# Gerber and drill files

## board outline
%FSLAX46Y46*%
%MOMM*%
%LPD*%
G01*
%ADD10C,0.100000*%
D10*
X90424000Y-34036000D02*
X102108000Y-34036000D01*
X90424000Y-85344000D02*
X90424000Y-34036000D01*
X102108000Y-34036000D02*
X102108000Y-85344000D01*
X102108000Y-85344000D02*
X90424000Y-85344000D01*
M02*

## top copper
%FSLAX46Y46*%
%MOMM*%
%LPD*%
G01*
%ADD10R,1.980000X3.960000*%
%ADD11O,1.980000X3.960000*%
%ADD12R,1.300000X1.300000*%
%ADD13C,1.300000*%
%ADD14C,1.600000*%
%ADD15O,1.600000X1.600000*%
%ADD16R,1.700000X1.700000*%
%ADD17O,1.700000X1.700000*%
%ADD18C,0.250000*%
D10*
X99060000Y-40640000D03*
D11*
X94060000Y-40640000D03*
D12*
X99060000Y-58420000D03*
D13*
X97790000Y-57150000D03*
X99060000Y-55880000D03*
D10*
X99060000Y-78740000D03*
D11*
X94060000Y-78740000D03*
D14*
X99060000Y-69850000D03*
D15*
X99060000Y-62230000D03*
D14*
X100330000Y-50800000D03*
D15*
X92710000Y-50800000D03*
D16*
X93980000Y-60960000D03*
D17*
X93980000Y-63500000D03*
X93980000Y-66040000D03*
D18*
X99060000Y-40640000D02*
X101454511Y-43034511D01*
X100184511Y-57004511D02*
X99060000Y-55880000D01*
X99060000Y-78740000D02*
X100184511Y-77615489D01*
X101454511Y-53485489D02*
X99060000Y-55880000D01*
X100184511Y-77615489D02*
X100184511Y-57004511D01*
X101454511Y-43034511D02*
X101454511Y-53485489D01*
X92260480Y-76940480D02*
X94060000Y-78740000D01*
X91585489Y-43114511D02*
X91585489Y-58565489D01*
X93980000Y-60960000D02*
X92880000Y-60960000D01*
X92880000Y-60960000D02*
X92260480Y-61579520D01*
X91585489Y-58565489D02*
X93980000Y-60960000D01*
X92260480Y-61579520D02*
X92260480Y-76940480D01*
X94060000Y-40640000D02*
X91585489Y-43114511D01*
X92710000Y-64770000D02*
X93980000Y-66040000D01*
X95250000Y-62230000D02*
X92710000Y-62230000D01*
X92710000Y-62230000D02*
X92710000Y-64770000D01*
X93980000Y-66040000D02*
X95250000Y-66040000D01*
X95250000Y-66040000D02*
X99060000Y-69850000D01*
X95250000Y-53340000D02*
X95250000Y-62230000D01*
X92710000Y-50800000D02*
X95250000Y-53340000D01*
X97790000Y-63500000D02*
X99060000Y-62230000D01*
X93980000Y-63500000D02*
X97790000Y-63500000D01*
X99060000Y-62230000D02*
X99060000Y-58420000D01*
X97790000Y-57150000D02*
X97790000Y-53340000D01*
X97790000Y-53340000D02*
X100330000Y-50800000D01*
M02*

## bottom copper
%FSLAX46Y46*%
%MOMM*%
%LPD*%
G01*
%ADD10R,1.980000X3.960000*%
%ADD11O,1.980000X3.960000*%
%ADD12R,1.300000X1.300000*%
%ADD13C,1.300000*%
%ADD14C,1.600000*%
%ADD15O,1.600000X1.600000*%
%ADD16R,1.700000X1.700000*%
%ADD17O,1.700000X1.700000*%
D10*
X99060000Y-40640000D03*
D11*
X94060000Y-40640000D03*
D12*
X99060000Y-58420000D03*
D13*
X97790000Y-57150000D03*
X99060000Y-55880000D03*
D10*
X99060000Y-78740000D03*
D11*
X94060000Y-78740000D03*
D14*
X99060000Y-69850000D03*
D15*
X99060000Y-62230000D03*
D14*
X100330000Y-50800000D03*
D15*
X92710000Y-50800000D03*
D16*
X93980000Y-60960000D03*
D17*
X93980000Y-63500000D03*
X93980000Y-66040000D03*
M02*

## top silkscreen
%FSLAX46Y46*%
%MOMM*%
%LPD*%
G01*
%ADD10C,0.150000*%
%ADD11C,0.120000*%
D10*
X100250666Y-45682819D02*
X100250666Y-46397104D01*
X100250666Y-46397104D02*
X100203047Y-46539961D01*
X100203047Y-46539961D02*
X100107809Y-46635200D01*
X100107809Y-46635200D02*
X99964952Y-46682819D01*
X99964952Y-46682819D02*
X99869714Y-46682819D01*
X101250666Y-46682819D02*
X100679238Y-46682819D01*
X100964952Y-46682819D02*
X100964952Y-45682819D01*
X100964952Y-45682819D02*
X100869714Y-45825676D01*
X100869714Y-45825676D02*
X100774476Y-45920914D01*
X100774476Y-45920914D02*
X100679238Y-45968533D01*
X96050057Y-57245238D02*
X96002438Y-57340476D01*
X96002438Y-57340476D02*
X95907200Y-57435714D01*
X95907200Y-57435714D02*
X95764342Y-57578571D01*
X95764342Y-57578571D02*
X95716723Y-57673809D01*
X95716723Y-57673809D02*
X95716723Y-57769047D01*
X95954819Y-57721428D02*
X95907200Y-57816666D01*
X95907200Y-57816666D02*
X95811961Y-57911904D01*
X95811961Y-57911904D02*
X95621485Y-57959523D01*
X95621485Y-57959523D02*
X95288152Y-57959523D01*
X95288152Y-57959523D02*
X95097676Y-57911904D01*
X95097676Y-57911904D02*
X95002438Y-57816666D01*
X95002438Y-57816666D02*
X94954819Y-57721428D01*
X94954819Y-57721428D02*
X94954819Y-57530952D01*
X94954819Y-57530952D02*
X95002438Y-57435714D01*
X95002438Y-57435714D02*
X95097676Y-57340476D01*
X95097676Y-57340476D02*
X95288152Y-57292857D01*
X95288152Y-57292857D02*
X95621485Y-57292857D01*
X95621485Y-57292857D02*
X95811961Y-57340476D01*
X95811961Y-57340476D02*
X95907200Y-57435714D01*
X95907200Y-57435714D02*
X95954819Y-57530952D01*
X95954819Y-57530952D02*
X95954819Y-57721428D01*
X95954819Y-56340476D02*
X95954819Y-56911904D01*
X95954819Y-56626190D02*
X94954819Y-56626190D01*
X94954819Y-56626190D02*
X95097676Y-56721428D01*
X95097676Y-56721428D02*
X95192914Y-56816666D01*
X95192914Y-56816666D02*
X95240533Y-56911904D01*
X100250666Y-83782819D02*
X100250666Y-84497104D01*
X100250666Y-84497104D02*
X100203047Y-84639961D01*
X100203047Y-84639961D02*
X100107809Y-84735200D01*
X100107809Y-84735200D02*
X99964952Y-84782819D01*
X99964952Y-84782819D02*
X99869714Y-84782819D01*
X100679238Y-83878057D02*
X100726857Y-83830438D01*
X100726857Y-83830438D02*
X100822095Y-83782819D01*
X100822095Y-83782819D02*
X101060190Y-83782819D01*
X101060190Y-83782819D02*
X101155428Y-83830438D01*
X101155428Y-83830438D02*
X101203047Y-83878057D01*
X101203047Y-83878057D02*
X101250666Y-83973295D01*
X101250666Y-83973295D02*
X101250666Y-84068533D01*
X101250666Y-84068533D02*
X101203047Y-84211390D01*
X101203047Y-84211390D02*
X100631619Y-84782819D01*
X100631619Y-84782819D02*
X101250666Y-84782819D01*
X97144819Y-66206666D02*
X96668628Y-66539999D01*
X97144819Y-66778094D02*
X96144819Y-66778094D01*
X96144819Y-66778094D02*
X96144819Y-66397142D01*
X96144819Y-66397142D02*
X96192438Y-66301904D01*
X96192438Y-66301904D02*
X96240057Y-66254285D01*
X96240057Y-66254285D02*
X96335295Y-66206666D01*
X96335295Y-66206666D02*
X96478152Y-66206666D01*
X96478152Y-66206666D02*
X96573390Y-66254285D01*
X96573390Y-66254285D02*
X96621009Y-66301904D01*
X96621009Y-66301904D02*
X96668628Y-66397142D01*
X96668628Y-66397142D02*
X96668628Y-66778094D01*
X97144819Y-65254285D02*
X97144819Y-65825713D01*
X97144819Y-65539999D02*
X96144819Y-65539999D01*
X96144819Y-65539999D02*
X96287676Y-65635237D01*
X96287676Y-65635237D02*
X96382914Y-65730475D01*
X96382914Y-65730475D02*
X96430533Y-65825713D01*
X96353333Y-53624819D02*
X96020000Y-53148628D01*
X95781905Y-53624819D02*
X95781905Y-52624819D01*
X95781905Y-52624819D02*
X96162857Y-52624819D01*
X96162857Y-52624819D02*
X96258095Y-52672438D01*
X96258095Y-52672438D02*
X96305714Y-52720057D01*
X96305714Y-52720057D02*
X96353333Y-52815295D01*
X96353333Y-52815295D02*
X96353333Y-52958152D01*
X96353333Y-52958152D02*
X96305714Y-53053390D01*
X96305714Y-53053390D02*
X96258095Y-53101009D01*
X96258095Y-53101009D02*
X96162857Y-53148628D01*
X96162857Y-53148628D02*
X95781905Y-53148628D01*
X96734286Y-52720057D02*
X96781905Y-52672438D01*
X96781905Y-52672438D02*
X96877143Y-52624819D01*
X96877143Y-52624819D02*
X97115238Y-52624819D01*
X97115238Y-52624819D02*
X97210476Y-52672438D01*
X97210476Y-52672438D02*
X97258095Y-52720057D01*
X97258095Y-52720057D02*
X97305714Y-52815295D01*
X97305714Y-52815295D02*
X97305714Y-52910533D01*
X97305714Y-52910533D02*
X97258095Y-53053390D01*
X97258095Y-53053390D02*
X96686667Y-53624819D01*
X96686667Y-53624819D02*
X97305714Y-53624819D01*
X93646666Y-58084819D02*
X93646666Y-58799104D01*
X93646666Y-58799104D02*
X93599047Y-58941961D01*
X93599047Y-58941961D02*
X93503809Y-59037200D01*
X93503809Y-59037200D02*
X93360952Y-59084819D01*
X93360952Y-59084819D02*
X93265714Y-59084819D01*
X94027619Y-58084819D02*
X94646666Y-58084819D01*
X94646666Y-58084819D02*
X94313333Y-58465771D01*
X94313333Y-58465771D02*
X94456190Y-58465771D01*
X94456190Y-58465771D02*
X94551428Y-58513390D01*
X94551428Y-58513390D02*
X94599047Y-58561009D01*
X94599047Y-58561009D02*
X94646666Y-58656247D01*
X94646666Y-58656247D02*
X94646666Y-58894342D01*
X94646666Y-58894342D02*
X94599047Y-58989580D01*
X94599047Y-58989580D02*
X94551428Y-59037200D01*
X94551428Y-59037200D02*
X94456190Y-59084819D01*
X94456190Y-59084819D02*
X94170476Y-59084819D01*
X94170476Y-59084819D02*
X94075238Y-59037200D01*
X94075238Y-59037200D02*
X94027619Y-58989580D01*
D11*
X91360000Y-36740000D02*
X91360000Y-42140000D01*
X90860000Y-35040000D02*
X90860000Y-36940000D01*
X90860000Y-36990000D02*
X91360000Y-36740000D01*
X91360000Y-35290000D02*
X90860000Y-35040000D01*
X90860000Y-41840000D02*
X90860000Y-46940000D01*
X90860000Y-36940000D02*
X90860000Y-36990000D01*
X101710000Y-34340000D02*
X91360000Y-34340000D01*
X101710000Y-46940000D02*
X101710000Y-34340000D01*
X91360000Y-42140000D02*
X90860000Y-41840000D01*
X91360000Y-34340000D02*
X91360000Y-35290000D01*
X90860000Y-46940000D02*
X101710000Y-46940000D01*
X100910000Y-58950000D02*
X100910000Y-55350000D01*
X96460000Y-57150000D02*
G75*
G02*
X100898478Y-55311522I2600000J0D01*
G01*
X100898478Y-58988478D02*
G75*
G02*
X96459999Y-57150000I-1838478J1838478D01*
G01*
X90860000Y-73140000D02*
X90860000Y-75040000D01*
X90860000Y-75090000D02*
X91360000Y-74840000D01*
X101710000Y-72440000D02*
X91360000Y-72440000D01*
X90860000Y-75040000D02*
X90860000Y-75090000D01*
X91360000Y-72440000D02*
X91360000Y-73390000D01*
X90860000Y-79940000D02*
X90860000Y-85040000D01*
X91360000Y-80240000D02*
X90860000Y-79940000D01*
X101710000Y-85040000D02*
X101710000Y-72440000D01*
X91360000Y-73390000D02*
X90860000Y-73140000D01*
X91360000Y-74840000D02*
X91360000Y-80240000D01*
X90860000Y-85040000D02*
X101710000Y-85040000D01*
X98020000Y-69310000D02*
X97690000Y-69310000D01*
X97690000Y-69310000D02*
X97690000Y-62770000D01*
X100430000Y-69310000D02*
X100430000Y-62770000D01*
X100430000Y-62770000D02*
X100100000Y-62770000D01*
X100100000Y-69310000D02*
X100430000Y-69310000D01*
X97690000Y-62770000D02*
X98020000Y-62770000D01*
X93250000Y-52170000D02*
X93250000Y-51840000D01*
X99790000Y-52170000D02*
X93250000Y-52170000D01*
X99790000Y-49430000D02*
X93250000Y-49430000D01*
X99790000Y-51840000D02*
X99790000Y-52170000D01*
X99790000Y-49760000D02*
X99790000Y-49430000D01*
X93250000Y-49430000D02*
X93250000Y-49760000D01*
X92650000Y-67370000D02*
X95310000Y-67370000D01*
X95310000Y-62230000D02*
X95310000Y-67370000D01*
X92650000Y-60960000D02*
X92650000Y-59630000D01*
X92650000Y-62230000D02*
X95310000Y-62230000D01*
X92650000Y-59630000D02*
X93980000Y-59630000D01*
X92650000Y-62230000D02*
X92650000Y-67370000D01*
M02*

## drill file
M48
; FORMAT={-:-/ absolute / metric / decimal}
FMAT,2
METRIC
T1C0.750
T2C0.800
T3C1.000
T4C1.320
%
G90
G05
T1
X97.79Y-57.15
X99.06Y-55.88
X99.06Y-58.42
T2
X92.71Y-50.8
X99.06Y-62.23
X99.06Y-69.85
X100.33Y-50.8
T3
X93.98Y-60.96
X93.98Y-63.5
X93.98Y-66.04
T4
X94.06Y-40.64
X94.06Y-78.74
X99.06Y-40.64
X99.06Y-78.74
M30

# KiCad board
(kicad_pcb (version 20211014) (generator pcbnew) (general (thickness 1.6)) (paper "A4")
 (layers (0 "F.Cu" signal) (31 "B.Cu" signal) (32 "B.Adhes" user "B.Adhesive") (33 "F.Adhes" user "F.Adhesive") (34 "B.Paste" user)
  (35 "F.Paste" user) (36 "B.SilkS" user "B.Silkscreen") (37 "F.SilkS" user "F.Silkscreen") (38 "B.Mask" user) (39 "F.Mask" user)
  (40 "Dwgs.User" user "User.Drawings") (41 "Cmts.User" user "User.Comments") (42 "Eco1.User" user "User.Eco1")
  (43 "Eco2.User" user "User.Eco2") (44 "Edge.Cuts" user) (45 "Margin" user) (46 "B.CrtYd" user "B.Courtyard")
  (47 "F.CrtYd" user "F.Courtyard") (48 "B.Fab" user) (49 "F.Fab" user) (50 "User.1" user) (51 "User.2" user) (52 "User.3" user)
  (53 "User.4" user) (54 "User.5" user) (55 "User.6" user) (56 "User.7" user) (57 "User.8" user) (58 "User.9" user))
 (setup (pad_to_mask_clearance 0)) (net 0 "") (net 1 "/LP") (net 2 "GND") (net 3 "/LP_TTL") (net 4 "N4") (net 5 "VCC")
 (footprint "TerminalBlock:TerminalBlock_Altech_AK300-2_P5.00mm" (layer "F.Cu") (at 99.06 40.64 180)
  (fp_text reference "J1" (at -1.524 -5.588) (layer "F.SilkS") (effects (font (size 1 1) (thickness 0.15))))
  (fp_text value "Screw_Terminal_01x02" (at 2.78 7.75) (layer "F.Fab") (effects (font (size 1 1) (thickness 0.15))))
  (fp_line (start 7.7 3.9) (end 7.7 -1.5) (layer "F.SilkS") (width 0.12))
  (fp_line (start 8.2 5.6) (end 8.2 3.7) (layer "F.SilkS") (width 0.12))
  (fp_line (start 8.2 3.65) (end 7.7 3.9) (layer "F.SilkS") (width 0.12))
  (fp_line (start 7.7 5.35) (end 8.2 5.6) (layer "F.SilkS") (width 0.12))
  (fp_line (start 8.2 -1.2) (end 8.2 -6.3) (layer "F.SilkS") (width 0.12))
  (fp_line (start 8.2 3.7) (end 8.2 3.65) (layer "F.SilkS") (width 0.12))
  (fp_line (start -2.65 6.3) (end 7.7 6.3) (layer "F.SilkS") (width 0.12))
  (fp_line (start -2.65 -6.3) (end -2.65 6.3) (layer "F.SilkS") (width 0.12))
  (fp_line (start 7.7 -1.5) (end 8.2 -1.2) (layer "F.SilkS") (width 0.12))
  (fp_line (start 7.7 6.3) (end 7.7 5.35) (layer "F.SilkS") (width 0.12))
  (fp_line (start 8.2 -6.3) (end -2.65 -6.3) (layer "F.SilkS") (width 0.12))
  (pad "1" thru_hole rect (at 0 0 180) (size 1.98 3.96) (drill 1.32) (layers *.Cu *.Mask) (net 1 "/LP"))
  (pad "2" thru_hole oval (at 5 0 180) (size 1.98 3.96) (drill 1.32) (layers *.Cu *.Mask) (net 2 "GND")))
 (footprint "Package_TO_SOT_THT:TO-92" (layer "F.Cu") (at 99.06 58.42 90)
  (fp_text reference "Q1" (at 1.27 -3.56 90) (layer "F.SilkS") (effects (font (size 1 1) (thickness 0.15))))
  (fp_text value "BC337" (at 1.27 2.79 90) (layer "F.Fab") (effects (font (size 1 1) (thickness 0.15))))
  (fp_line (start -0.53 1.85) (end 3.07 1.85) (layer "F.SilkS") (width 0.12))
  (fp_arc (start 1.27 -2.6) (mid 3.672087 -0.994977) (end 3.108478 1.838478) (layer "F.SilkS") (width 0.12))
  (fp_arc (start -0.568478 1.838478) (mid -1.132087 -0.994977) (end 1.27 -2.6) (layer "F.SilkS") (width 0.12))
  (pad "1" thru_hole rect (at 0 0 90) (size 1.3 1.3) (drill 0.75) (layers *.Cu *.Mask) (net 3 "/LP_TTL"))
  (pad "2" thru_hole circle (at 1.27 -1.27 90) (size 1.3 1.3) (drill 0.75) (layers *.Cu *.Mask) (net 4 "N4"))
  (pad "3" thru_hole circle (at 2.54 0 90) (size 1.3 1.3) (drill 0.75) (layers *.Cu *.Mask) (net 1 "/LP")))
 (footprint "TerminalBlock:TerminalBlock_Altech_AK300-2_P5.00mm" (layer "F.Cu") (at 99.06 78.74 180)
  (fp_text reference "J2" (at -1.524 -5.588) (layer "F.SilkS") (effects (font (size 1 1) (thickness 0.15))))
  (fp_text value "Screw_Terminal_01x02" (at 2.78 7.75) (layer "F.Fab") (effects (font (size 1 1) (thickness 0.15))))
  (fp_line (start 8.2 5.6) (end 8.2 3.7) (layer "F.SilkS") (width 0.12))
  (fp_line (start 8.2 3.65) (end 7.7 3.9) (layer "F.SilkS") (width 0.12))
  (fp_line (start -2.65 6.3) (end 7.7 6.3) (layer "F.SilkS") (width 0.12))
  (fp_line (start 8.2 3.7) (end 8.2 3.65) (layer "F.SilkS") (width 0.12))
  (fp_line (start 7.7 6.3) (end 7.7 5.35) (layer "F.SilkS") (width 0.12))
  (fp_line (start 8.2 -1.2) (end 8.2 -6.3) (layer "F.SilkS") (width 0.12))
  (fp_line (start 7.7 -1.5) (end 8.2 -1.2) (layer "F.SilkS") (width 0.12))
  (fp_line (start -2.65 -6.3) (end -2.65 6.3) (layer "F.SilkS") (width 0.12))
  (fp_line (start 7.7 5.35) (end 8.2 5.6) (layer "F.SilkS") (width 0.12))
  (fp_line (start 7.7 3.9) (end 7.7 -1.5) (layer "F.SilkS") (width 0.12))
  (fp_line (start 8.2 -6.3) (end -2.65 -6.3) (layer "F.SilkS") (width 0.12))
  (pad "1" thru_hole rect (at 0 0 180) (size 1.98 3.96) (drill 1.32) (layers *.Cu *.Mask) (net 1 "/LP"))
  (pad "2" thru_hole oval (at 5 0 180) (size 1.98 3.96) (drill 1.32) (layers *.Cu *.Mask) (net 2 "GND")))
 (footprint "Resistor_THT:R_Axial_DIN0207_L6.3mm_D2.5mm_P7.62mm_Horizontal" (layer "F.Cu") (at 99.06 69.85 90)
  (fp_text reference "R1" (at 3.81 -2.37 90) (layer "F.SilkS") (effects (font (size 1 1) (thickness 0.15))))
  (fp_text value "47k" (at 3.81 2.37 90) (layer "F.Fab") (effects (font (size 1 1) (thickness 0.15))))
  (fp_line (start 0.54 -1.04) (end 0.54 -1.37) (layer "F.SilkS") (width 0.12))
  (fp_line (start 0.54 -1.37) (end 7.08 -1.37) (layer "F.SilkS") (width 0.12))
  (fp_line (start 0.54 1.37) (end 7.08 1.37) (layer "F.SilkS") (width 0.12))
  (fp_line (start 7.08 1.37) (end 7.08 1.04) (layer "F.SilkS") (width 0.12))
  (fp_line (start 0.54 1.04) (end 0.54 1.37) (layer "F.SilkS") (width 0.12))
  (fp_line (start 7.08 -1.37) (end 7.08 -1.04) (layer "F.SilkS") (width 0.12))
  (pad "1" thru_hole circle (at 0 0 90) (size 1.6 1.6) (drill 0.8) (layers *.Cu *.Mask) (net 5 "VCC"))
  (pad "2" thru_hole oval (at 7.62 0 90) (size 1.6 1.6) (drill 0.8) (layers *.Cu *.Mask) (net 3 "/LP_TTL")))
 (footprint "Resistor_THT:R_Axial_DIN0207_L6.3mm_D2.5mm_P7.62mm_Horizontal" (layer "F.Cu") (at 100.33 50.8 180)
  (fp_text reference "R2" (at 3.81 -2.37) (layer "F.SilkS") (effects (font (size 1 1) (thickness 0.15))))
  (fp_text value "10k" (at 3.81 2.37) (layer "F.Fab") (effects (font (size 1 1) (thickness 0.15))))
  (fp_line (start 7.08 -1.37) (end 7.08 -1.04) (layer "F.SilkS") (width 0.12))
  (fp_line (start 0.54 -1.37) (end 7.08 -1.37) (layer "F.SilkS") (width 0.12))
  (fp_line (start 0.54 1.37) (end 7.08 1.37) (layer "F.SilkS") (width 0.12))
  (fp_line (start 0.54 -1.04) (end 0.54 -1.37) (layer "F.SilkS") (width 0.12))
  (fp_line (start 0.54 1.04) (end 0.54 1.37) (layer "F.SilkS") (width 0.12))
  (fp_line (start 7.08 1.37) (end 7.08 1.04) (layer "F.SilkS") (width 0.12))
  (pad "1" thru_hole circle (at 0 0 180) (size 1.6 1.6) (drill 0.8) (layers *.Cu *.Mask) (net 4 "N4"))
  (pad "2" thru_hole oval (at 7.62 0 180) (size 1.6 1.6) (drill 0.8) (layers *.Cu *.Mask) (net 5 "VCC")))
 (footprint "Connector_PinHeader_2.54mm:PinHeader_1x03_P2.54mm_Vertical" (layer "F.Cu") (at 93.98 60.96)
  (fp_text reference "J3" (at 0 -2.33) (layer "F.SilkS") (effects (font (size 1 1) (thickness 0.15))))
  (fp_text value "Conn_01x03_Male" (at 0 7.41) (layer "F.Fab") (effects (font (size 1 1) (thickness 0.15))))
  (fp_line (start -1.33 6.41) (end 1.33 6.41) (layer "F.SilkS") (width 0.12))
  (fp_line (start 1.33 1.27) (end 1.33 6.41) (layer "F.SilkS") (width 0.12))
  (fp_line (start -1.33 0) (end -1.33 -1.33) (layer "F.SilkS") (width 0.12))
  (fp_line (start -1.33 1.27) (end 1.33 1.27) (layer "F.SilkS") (width 0.12))
  (fp_line (start -1.33 -1.33) (end 0 -1.33) (layer "F.SilkS") (width 0.12))
  (fp_line (start -1.33 1.27) (end -1.33 6.41) (layer "F.SilkS") (width 0.12))
  (pad "1" thru_hole rect (at 0 0) (size 1.7 1.7) (drill 1) (layers *.Cu *.Mask) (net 2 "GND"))
  (pad "2" thru_hole oval (at 0 2.54) (size 1.7 1.7) (drill 1) (layers *.Cu *.Mask) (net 3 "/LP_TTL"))
  (pad "3" thru_hole oval (at 0 5.08) (size 1.7 1.7) (drill 1) (layers *.Cu *.Mask) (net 5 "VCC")))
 (gr_line (start 90.424 34.036) (end 102.108 34.036) (layer "Edge.Cuts") (width 0.1))
 (gr_line (start 90.424 85.344) (end 90.424 34.036) (layer "Edge.Cuts") (width 0.1))
 (gr_line (start 102.108 34.036) (end 102.108 85.344) (layer "Edge.Cuts") (width 0.1))
 (gr_line (start 102.108 85.344) (end 90.424 85.344) (layer "Edge.Cuts") (width 0.1))
 (segment (start 99.06 40.64) (end 101.454511 43.034511) (width 0.25) (layer "F.Cu") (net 1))
 (segment (start 100.184511 57.004511) (end 99.06 55.88) (width 0.25) (layer "F.Cu") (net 1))
 (segment (start 99.06 78.74) (end 100.184511 77.615489) (width 0.25) (layer "F.Cu") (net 1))
 (segment (start 101.454511 53.485489) (end 99.06 55.88) (width 0.25) (layer "F.Cu") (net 1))
 (segment (start 100.184511 77.615489) (end 100.184511 57.004511) (width 0.25) (layer "F.Cu") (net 1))
 (segment (start 101.454511 43.034511) (end 101.454511 53.485489) (width 0.25) (layer "F.Cu") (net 1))
 (segment (start 92.26048 76.94048) (end 94.06 78.74) (width 0.25) (layer "F.Cu") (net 2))
 (segment (start 91.585489 43.114511) (end 91.585489 58.565489) (width 0.25) (layer "F.Cu") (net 2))
 (segment (start 93.98 60.96) (end 92.88 60.96) (width 0.25) (layer "F.Cu") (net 2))
 (segment (start 92.88 60.96) (end 92.26048 61.57952) (width 0.25) (layer "F.Cu") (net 2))
 (segment (start 91.585489 58.565489) (end 93.98 60.96) (width 0.25) (layer "F.Cu") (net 2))
 (segment (start 92.26048 61.57952) (end 92.26048 76.94048) (width 0.25) (layer "F.Cu") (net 2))
 (segment (start 94.06 40.64) (end 91.585489 43.114511) (width 0.25) (layer "F.Cu") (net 2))
 (segment (start 92.71 64.77) (end 93.98 66.04) (width 0.25) (layer "F.Cu") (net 5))
 (segment (start 95.25 62.23) (end 92.71 62.23) (width 0.25) (layer "F.Cu") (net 5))
 (segment (start 92.71 62.23) (end 92.71 64.77) (width 0.25) (layer "F.Cu") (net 5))
 (segment (start 93.98 66.04) (end 95.25 66.04) (width 0.25) (layer "F.Cu") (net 5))
 (segment (start 95.25 66.04) (end 99.06 69.85) (width 0.25) (layer "F.Cu") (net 5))
 (segment (start 95.25 53.34) (end 95.25 62.23) (width 0.25) (layer "F.Cu") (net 5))
 (segment (start 92.71 50.8) (end 95.25 53.34) (width 0.25) (layer "F.Cu") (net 5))
 (segment (start 97.79 63.5) (end 99.06 62.23) (width 0.25) (layer "F.Cu") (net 3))
 (segment (start 93.98 63.5) (end 97.79 63.5) (width 0.25) (layer "F.Cu") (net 3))
 (segment (start 99.06 62.23) (end 99.06 58.42) (width 0.25) (layer "F.Cu") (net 3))
 (segment (start 97.79 57.15) (end 97.79 53.34) (width 0.25) (layer "F.Cu") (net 4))
 (segment (start 97.79 53.34) (end 100.33 50.8) (width 0.25) (layer "F.Cu") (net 4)))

